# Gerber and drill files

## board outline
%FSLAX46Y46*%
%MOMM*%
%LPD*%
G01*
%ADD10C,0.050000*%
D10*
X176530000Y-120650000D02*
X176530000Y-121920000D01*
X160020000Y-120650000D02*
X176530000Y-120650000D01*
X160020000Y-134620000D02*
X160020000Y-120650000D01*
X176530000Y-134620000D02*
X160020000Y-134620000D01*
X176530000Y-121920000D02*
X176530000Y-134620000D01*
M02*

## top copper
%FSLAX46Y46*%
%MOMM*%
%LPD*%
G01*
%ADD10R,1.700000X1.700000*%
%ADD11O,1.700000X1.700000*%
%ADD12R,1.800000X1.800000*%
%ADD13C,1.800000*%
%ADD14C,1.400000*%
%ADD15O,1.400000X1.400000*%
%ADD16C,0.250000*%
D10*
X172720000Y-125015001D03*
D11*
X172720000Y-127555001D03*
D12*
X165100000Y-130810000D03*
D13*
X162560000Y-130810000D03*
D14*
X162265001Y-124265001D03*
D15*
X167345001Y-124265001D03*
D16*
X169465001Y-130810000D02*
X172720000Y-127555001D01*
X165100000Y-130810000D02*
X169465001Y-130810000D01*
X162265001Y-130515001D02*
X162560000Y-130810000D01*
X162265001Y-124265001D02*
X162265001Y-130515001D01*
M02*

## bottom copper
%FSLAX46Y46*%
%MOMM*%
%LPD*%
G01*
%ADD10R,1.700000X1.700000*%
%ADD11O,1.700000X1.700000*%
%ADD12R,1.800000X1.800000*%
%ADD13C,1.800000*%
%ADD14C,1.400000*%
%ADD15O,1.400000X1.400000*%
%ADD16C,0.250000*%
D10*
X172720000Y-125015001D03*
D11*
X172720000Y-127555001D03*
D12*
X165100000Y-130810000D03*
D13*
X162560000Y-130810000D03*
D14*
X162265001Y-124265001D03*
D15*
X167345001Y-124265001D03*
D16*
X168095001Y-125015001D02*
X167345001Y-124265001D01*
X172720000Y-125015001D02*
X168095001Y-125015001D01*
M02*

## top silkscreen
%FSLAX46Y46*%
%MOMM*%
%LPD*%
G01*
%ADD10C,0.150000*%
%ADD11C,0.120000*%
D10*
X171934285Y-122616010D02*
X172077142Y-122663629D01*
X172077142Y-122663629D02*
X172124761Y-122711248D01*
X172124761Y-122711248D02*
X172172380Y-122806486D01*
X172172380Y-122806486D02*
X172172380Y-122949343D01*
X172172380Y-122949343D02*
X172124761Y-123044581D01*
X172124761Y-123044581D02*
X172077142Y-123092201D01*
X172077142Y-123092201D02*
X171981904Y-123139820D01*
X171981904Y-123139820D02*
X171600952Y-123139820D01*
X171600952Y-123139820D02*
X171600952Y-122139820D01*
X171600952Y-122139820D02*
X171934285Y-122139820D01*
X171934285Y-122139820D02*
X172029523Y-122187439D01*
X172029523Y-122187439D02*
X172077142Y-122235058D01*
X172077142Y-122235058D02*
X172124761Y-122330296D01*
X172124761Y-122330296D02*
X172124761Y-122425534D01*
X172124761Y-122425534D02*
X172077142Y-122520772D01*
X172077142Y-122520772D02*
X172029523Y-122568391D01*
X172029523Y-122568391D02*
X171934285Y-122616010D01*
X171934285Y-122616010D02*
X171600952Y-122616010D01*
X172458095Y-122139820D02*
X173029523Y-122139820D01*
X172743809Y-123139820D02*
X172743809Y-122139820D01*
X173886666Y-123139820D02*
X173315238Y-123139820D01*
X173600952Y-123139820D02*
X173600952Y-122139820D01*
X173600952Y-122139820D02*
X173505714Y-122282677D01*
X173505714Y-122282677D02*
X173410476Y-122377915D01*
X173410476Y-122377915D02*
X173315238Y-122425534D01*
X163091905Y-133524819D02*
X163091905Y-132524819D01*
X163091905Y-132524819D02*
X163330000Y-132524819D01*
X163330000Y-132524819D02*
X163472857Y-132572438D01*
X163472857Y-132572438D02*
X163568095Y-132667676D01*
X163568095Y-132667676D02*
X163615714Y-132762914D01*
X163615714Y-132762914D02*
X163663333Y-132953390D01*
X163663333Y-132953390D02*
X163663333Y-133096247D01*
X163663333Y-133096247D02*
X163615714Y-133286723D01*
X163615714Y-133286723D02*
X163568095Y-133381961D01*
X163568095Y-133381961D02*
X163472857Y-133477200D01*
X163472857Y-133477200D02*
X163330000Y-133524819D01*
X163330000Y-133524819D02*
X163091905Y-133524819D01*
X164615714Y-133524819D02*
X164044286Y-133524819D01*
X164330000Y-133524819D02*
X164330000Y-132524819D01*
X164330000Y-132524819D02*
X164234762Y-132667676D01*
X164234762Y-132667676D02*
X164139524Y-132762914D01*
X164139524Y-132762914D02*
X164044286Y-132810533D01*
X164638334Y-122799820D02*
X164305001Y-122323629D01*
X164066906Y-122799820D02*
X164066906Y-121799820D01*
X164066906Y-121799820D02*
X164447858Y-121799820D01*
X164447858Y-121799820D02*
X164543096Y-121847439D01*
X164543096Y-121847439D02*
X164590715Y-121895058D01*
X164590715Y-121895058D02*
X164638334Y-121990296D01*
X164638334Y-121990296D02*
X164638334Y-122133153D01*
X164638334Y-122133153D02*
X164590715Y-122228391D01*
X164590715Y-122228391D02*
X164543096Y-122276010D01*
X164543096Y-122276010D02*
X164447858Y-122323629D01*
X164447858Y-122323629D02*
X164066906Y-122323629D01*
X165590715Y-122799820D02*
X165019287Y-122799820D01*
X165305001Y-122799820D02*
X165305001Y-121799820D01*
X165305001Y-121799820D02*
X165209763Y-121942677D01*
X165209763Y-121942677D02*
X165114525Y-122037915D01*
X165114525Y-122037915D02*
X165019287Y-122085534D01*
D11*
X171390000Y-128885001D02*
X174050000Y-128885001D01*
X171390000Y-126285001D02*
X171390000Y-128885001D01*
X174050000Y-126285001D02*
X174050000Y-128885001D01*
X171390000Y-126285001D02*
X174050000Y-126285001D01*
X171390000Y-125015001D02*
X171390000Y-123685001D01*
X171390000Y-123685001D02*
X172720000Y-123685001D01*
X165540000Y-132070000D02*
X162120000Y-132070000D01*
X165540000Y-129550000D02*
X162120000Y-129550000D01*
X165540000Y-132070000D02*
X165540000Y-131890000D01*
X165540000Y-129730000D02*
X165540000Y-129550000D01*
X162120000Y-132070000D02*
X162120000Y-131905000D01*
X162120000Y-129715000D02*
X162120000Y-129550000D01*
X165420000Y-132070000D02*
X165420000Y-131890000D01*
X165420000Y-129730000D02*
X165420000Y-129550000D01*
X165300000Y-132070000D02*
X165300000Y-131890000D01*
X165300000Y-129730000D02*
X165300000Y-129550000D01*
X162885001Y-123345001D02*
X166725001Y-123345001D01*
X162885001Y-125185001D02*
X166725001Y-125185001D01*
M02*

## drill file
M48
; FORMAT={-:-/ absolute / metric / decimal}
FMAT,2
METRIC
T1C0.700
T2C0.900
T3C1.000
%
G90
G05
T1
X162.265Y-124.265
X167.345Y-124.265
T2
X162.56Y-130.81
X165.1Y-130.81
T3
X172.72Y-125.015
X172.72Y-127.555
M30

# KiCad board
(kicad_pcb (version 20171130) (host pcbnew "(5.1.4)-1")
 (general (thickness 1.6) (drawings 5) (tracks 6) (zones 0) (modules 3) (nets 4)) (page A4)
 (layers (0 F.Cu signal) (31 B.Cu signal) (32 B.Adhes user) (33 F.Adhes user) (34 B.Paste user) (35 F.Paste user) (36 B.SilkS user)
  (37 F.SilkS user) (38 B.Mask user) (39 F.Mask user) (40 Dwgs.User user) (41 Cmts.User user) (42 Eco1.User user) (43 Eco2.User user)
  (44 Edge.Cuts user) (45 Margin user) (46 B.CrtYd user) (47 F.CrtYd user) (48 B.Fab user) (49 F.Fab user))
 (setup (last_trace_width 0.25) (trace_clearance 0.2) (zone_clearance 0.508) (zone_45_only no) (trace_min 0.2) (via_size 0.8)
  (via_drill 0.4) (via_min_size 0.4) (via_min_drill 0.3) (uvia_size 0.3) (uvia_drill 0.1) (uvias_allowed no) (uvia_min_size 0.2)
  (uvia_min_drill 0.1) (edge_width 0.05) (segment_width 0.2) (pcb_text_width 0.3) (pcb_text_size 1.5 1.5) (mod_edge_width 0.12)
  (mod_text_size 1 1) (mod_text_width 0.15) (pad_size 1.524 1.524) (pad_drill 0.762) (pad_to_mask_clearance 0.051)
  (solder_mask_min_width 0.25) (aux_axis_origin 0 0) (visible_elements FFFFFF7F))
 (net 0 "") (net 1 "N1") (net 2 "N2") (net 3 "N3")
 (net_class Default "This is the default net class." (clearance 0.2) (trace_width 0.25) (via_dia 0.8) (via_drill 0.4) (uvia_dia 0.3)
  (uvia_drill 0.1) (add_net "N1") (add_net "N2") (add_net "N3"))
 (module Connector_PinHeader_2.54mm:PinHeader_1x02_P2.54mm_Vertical (layer F.Cu) (at 172.72 125.015001)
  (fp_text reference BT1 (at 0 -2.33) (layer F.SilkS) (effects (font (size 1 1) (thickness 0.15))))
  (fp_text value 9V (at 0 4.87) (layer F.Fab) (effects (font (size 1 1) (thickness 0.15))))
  (fp_line (start -1.33 3.87) (end 1.33 3.87) (layer F.SilkS) (width 0.12))
  (fp_line (start -1.33 1.27) (end -1.33 3.87) (layer F.SilkS) (width 0.12))
  (fp_line (start 1.33 1.27) (end 1.33 3.87) (layer F.SilkS) (width 0.12))
  (fp_line (start -1.33 1.27) (end 1.33 1.27) (layer F.SilkS) (width 0.12))
  (fp_line (start -1.33 0) (end -1.33 -1.33) (layer F.SilkS) (width 0.12))
  (fp_line (start -1.33 -1.33) (end 0 -1.33) (layer F.SilkS) (width 0.12))
  (pad 1 thru_hole rect (at 0 0) (size 1.7 1.7) (drill 1) (layers *.Cu *.Mask) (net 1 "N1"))
  (pad 2 thru_hole oval (at 0 2.54) (size 1.7 1.7) (drill 1) (layers *.Cu *.Mask) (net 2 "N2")))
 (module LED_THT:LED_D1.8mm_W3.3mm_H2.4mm (layer F.Cu) (at 165.1 130.81 180)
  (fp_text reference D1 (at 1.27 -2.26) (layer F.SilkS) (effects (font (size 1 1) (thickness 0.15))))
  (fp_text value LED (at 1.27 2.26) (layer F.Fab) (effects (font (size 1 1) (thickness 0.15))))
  (fp_line (start -0.44 -1.26) (end 2.98 -1.26) (layer F.SilkS) (width 0.12))
  (fp_line (start -0.44 1.26) (end 2.98 1.26) (layer F.SilkS) (width 0.12))
  (fp_line (start -0.44 -1.26) (end -0.44 -1.08) (layer F.SilkS) (width 0.12))
  (fp_line (start -0.44 1.08) (end -0.44 1.26) (layer F.SilkS) (width 0.12))
  (fp_line (start 2.98 -1.26) (end 2.98 -1.095) (layer F.SilkS) (width 0.12))
  (fp_line (start 2.98 1.095) (end 2.98 1.26) (layer F.SilkS) (width 0.12))
  (fp_line (start -0.32 -1.26) (end -0.32 -1.08) (layer F.SilkS) (width 0.12))
  (fp_line (start -0.32 1.08) (end -0.32 1.26) (layer F.SilkS) (width 0.12))
  (fp_line (start -0.2 -1.26) (end -0.2 -1.08) (layer F.SilkS) (width 0.12))
  (fp_line (start -0.2 1.08) (end -0.2 1.26) (layer F.SilkS) (width 0.12))
  (pad 1 thru_hole rect (at 0 0 180) (size 1.8 1.8) (drill 0.9) (layers *.Cu *.Mask) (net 2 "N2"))
  (pad 2 thru_hole circle (at 2.54 0 180) (size 1.8 1.8) (drill 0.9) (layers *.Cu *.Mask) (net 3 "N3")))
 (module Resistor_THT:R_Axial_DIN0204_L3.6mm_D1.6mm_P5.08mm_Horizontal (layer F.Cu) (at 162.265001 124.265001)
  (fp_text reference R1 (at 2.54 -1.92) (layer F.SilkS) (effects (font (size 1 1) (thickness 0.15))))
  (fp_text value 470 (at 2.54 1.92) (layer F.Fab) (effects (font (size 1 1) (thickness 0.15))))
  (fp_line (start 0.62 -0.92) (end 4.46 -0.92) (layer F.SilkS) (width 0.12))
  (fp_line (start 0.62 0.92) (end 4.46 0.92) (layer F.SilkS) (width 0.12))
  (pad 1 thru_hole circle (at 0 0) (size 1.4 1.4) (drill 0.7) (layers *.Cu *.Mask) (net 3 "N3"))
  (pad 2 thru_hole oval (at 5.08 0) (size 1.4 1.4) (drill 0.7) (layers *.Cu *.Mask) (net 1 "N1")))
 (gr_line (start 176.53 120.65) (end 176.53 121.92) (layer Edge.Cuts) (width 0.05))
 (gr_line (start 160.02 120.65) (end 176.53 120.65) (layer Edge.Cuts) (width 0.05))
 (gr_line (start 160.02 134.62) (end 160.02 120.65) (layer Edge.Cuts) (width 0.05))
 (gr_line (start 176.53 134.62) (end 160.02 134.62) (layer Edge.Cuts) (width 0.05))
 (gr_line (start 176.53 121.92) (end 176.53 134.62) (layer Edge.Cuts) (width 0.05))
 (segment (start 168.095001 125.015001) (end 167.345001 124.265001) (width 0.25) (layer B.Cu) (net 1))
 (segment (start 172.72 125.015001) (end 168.095001 125.015001) (width 0.25) (layer B.Cu) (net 1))
 (segment (start 169.465001 130.81) (end 172.72 127.555001) (width 0.25) (layer F.Cu) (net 2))
 (segment (start 165.1 130.81) (end 169.465001 130.81) (width 0.25) (layer F.Cu) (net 2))
 (segment (start 162.265001 130.515001) (end 162.56 130.81) (width 0.25) (layer F.Cu) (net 3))
 (segment (start 162.265001 124.265001) (end 162.265001 130.515001) (width 0.25) (layer F.Cu) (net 3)))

